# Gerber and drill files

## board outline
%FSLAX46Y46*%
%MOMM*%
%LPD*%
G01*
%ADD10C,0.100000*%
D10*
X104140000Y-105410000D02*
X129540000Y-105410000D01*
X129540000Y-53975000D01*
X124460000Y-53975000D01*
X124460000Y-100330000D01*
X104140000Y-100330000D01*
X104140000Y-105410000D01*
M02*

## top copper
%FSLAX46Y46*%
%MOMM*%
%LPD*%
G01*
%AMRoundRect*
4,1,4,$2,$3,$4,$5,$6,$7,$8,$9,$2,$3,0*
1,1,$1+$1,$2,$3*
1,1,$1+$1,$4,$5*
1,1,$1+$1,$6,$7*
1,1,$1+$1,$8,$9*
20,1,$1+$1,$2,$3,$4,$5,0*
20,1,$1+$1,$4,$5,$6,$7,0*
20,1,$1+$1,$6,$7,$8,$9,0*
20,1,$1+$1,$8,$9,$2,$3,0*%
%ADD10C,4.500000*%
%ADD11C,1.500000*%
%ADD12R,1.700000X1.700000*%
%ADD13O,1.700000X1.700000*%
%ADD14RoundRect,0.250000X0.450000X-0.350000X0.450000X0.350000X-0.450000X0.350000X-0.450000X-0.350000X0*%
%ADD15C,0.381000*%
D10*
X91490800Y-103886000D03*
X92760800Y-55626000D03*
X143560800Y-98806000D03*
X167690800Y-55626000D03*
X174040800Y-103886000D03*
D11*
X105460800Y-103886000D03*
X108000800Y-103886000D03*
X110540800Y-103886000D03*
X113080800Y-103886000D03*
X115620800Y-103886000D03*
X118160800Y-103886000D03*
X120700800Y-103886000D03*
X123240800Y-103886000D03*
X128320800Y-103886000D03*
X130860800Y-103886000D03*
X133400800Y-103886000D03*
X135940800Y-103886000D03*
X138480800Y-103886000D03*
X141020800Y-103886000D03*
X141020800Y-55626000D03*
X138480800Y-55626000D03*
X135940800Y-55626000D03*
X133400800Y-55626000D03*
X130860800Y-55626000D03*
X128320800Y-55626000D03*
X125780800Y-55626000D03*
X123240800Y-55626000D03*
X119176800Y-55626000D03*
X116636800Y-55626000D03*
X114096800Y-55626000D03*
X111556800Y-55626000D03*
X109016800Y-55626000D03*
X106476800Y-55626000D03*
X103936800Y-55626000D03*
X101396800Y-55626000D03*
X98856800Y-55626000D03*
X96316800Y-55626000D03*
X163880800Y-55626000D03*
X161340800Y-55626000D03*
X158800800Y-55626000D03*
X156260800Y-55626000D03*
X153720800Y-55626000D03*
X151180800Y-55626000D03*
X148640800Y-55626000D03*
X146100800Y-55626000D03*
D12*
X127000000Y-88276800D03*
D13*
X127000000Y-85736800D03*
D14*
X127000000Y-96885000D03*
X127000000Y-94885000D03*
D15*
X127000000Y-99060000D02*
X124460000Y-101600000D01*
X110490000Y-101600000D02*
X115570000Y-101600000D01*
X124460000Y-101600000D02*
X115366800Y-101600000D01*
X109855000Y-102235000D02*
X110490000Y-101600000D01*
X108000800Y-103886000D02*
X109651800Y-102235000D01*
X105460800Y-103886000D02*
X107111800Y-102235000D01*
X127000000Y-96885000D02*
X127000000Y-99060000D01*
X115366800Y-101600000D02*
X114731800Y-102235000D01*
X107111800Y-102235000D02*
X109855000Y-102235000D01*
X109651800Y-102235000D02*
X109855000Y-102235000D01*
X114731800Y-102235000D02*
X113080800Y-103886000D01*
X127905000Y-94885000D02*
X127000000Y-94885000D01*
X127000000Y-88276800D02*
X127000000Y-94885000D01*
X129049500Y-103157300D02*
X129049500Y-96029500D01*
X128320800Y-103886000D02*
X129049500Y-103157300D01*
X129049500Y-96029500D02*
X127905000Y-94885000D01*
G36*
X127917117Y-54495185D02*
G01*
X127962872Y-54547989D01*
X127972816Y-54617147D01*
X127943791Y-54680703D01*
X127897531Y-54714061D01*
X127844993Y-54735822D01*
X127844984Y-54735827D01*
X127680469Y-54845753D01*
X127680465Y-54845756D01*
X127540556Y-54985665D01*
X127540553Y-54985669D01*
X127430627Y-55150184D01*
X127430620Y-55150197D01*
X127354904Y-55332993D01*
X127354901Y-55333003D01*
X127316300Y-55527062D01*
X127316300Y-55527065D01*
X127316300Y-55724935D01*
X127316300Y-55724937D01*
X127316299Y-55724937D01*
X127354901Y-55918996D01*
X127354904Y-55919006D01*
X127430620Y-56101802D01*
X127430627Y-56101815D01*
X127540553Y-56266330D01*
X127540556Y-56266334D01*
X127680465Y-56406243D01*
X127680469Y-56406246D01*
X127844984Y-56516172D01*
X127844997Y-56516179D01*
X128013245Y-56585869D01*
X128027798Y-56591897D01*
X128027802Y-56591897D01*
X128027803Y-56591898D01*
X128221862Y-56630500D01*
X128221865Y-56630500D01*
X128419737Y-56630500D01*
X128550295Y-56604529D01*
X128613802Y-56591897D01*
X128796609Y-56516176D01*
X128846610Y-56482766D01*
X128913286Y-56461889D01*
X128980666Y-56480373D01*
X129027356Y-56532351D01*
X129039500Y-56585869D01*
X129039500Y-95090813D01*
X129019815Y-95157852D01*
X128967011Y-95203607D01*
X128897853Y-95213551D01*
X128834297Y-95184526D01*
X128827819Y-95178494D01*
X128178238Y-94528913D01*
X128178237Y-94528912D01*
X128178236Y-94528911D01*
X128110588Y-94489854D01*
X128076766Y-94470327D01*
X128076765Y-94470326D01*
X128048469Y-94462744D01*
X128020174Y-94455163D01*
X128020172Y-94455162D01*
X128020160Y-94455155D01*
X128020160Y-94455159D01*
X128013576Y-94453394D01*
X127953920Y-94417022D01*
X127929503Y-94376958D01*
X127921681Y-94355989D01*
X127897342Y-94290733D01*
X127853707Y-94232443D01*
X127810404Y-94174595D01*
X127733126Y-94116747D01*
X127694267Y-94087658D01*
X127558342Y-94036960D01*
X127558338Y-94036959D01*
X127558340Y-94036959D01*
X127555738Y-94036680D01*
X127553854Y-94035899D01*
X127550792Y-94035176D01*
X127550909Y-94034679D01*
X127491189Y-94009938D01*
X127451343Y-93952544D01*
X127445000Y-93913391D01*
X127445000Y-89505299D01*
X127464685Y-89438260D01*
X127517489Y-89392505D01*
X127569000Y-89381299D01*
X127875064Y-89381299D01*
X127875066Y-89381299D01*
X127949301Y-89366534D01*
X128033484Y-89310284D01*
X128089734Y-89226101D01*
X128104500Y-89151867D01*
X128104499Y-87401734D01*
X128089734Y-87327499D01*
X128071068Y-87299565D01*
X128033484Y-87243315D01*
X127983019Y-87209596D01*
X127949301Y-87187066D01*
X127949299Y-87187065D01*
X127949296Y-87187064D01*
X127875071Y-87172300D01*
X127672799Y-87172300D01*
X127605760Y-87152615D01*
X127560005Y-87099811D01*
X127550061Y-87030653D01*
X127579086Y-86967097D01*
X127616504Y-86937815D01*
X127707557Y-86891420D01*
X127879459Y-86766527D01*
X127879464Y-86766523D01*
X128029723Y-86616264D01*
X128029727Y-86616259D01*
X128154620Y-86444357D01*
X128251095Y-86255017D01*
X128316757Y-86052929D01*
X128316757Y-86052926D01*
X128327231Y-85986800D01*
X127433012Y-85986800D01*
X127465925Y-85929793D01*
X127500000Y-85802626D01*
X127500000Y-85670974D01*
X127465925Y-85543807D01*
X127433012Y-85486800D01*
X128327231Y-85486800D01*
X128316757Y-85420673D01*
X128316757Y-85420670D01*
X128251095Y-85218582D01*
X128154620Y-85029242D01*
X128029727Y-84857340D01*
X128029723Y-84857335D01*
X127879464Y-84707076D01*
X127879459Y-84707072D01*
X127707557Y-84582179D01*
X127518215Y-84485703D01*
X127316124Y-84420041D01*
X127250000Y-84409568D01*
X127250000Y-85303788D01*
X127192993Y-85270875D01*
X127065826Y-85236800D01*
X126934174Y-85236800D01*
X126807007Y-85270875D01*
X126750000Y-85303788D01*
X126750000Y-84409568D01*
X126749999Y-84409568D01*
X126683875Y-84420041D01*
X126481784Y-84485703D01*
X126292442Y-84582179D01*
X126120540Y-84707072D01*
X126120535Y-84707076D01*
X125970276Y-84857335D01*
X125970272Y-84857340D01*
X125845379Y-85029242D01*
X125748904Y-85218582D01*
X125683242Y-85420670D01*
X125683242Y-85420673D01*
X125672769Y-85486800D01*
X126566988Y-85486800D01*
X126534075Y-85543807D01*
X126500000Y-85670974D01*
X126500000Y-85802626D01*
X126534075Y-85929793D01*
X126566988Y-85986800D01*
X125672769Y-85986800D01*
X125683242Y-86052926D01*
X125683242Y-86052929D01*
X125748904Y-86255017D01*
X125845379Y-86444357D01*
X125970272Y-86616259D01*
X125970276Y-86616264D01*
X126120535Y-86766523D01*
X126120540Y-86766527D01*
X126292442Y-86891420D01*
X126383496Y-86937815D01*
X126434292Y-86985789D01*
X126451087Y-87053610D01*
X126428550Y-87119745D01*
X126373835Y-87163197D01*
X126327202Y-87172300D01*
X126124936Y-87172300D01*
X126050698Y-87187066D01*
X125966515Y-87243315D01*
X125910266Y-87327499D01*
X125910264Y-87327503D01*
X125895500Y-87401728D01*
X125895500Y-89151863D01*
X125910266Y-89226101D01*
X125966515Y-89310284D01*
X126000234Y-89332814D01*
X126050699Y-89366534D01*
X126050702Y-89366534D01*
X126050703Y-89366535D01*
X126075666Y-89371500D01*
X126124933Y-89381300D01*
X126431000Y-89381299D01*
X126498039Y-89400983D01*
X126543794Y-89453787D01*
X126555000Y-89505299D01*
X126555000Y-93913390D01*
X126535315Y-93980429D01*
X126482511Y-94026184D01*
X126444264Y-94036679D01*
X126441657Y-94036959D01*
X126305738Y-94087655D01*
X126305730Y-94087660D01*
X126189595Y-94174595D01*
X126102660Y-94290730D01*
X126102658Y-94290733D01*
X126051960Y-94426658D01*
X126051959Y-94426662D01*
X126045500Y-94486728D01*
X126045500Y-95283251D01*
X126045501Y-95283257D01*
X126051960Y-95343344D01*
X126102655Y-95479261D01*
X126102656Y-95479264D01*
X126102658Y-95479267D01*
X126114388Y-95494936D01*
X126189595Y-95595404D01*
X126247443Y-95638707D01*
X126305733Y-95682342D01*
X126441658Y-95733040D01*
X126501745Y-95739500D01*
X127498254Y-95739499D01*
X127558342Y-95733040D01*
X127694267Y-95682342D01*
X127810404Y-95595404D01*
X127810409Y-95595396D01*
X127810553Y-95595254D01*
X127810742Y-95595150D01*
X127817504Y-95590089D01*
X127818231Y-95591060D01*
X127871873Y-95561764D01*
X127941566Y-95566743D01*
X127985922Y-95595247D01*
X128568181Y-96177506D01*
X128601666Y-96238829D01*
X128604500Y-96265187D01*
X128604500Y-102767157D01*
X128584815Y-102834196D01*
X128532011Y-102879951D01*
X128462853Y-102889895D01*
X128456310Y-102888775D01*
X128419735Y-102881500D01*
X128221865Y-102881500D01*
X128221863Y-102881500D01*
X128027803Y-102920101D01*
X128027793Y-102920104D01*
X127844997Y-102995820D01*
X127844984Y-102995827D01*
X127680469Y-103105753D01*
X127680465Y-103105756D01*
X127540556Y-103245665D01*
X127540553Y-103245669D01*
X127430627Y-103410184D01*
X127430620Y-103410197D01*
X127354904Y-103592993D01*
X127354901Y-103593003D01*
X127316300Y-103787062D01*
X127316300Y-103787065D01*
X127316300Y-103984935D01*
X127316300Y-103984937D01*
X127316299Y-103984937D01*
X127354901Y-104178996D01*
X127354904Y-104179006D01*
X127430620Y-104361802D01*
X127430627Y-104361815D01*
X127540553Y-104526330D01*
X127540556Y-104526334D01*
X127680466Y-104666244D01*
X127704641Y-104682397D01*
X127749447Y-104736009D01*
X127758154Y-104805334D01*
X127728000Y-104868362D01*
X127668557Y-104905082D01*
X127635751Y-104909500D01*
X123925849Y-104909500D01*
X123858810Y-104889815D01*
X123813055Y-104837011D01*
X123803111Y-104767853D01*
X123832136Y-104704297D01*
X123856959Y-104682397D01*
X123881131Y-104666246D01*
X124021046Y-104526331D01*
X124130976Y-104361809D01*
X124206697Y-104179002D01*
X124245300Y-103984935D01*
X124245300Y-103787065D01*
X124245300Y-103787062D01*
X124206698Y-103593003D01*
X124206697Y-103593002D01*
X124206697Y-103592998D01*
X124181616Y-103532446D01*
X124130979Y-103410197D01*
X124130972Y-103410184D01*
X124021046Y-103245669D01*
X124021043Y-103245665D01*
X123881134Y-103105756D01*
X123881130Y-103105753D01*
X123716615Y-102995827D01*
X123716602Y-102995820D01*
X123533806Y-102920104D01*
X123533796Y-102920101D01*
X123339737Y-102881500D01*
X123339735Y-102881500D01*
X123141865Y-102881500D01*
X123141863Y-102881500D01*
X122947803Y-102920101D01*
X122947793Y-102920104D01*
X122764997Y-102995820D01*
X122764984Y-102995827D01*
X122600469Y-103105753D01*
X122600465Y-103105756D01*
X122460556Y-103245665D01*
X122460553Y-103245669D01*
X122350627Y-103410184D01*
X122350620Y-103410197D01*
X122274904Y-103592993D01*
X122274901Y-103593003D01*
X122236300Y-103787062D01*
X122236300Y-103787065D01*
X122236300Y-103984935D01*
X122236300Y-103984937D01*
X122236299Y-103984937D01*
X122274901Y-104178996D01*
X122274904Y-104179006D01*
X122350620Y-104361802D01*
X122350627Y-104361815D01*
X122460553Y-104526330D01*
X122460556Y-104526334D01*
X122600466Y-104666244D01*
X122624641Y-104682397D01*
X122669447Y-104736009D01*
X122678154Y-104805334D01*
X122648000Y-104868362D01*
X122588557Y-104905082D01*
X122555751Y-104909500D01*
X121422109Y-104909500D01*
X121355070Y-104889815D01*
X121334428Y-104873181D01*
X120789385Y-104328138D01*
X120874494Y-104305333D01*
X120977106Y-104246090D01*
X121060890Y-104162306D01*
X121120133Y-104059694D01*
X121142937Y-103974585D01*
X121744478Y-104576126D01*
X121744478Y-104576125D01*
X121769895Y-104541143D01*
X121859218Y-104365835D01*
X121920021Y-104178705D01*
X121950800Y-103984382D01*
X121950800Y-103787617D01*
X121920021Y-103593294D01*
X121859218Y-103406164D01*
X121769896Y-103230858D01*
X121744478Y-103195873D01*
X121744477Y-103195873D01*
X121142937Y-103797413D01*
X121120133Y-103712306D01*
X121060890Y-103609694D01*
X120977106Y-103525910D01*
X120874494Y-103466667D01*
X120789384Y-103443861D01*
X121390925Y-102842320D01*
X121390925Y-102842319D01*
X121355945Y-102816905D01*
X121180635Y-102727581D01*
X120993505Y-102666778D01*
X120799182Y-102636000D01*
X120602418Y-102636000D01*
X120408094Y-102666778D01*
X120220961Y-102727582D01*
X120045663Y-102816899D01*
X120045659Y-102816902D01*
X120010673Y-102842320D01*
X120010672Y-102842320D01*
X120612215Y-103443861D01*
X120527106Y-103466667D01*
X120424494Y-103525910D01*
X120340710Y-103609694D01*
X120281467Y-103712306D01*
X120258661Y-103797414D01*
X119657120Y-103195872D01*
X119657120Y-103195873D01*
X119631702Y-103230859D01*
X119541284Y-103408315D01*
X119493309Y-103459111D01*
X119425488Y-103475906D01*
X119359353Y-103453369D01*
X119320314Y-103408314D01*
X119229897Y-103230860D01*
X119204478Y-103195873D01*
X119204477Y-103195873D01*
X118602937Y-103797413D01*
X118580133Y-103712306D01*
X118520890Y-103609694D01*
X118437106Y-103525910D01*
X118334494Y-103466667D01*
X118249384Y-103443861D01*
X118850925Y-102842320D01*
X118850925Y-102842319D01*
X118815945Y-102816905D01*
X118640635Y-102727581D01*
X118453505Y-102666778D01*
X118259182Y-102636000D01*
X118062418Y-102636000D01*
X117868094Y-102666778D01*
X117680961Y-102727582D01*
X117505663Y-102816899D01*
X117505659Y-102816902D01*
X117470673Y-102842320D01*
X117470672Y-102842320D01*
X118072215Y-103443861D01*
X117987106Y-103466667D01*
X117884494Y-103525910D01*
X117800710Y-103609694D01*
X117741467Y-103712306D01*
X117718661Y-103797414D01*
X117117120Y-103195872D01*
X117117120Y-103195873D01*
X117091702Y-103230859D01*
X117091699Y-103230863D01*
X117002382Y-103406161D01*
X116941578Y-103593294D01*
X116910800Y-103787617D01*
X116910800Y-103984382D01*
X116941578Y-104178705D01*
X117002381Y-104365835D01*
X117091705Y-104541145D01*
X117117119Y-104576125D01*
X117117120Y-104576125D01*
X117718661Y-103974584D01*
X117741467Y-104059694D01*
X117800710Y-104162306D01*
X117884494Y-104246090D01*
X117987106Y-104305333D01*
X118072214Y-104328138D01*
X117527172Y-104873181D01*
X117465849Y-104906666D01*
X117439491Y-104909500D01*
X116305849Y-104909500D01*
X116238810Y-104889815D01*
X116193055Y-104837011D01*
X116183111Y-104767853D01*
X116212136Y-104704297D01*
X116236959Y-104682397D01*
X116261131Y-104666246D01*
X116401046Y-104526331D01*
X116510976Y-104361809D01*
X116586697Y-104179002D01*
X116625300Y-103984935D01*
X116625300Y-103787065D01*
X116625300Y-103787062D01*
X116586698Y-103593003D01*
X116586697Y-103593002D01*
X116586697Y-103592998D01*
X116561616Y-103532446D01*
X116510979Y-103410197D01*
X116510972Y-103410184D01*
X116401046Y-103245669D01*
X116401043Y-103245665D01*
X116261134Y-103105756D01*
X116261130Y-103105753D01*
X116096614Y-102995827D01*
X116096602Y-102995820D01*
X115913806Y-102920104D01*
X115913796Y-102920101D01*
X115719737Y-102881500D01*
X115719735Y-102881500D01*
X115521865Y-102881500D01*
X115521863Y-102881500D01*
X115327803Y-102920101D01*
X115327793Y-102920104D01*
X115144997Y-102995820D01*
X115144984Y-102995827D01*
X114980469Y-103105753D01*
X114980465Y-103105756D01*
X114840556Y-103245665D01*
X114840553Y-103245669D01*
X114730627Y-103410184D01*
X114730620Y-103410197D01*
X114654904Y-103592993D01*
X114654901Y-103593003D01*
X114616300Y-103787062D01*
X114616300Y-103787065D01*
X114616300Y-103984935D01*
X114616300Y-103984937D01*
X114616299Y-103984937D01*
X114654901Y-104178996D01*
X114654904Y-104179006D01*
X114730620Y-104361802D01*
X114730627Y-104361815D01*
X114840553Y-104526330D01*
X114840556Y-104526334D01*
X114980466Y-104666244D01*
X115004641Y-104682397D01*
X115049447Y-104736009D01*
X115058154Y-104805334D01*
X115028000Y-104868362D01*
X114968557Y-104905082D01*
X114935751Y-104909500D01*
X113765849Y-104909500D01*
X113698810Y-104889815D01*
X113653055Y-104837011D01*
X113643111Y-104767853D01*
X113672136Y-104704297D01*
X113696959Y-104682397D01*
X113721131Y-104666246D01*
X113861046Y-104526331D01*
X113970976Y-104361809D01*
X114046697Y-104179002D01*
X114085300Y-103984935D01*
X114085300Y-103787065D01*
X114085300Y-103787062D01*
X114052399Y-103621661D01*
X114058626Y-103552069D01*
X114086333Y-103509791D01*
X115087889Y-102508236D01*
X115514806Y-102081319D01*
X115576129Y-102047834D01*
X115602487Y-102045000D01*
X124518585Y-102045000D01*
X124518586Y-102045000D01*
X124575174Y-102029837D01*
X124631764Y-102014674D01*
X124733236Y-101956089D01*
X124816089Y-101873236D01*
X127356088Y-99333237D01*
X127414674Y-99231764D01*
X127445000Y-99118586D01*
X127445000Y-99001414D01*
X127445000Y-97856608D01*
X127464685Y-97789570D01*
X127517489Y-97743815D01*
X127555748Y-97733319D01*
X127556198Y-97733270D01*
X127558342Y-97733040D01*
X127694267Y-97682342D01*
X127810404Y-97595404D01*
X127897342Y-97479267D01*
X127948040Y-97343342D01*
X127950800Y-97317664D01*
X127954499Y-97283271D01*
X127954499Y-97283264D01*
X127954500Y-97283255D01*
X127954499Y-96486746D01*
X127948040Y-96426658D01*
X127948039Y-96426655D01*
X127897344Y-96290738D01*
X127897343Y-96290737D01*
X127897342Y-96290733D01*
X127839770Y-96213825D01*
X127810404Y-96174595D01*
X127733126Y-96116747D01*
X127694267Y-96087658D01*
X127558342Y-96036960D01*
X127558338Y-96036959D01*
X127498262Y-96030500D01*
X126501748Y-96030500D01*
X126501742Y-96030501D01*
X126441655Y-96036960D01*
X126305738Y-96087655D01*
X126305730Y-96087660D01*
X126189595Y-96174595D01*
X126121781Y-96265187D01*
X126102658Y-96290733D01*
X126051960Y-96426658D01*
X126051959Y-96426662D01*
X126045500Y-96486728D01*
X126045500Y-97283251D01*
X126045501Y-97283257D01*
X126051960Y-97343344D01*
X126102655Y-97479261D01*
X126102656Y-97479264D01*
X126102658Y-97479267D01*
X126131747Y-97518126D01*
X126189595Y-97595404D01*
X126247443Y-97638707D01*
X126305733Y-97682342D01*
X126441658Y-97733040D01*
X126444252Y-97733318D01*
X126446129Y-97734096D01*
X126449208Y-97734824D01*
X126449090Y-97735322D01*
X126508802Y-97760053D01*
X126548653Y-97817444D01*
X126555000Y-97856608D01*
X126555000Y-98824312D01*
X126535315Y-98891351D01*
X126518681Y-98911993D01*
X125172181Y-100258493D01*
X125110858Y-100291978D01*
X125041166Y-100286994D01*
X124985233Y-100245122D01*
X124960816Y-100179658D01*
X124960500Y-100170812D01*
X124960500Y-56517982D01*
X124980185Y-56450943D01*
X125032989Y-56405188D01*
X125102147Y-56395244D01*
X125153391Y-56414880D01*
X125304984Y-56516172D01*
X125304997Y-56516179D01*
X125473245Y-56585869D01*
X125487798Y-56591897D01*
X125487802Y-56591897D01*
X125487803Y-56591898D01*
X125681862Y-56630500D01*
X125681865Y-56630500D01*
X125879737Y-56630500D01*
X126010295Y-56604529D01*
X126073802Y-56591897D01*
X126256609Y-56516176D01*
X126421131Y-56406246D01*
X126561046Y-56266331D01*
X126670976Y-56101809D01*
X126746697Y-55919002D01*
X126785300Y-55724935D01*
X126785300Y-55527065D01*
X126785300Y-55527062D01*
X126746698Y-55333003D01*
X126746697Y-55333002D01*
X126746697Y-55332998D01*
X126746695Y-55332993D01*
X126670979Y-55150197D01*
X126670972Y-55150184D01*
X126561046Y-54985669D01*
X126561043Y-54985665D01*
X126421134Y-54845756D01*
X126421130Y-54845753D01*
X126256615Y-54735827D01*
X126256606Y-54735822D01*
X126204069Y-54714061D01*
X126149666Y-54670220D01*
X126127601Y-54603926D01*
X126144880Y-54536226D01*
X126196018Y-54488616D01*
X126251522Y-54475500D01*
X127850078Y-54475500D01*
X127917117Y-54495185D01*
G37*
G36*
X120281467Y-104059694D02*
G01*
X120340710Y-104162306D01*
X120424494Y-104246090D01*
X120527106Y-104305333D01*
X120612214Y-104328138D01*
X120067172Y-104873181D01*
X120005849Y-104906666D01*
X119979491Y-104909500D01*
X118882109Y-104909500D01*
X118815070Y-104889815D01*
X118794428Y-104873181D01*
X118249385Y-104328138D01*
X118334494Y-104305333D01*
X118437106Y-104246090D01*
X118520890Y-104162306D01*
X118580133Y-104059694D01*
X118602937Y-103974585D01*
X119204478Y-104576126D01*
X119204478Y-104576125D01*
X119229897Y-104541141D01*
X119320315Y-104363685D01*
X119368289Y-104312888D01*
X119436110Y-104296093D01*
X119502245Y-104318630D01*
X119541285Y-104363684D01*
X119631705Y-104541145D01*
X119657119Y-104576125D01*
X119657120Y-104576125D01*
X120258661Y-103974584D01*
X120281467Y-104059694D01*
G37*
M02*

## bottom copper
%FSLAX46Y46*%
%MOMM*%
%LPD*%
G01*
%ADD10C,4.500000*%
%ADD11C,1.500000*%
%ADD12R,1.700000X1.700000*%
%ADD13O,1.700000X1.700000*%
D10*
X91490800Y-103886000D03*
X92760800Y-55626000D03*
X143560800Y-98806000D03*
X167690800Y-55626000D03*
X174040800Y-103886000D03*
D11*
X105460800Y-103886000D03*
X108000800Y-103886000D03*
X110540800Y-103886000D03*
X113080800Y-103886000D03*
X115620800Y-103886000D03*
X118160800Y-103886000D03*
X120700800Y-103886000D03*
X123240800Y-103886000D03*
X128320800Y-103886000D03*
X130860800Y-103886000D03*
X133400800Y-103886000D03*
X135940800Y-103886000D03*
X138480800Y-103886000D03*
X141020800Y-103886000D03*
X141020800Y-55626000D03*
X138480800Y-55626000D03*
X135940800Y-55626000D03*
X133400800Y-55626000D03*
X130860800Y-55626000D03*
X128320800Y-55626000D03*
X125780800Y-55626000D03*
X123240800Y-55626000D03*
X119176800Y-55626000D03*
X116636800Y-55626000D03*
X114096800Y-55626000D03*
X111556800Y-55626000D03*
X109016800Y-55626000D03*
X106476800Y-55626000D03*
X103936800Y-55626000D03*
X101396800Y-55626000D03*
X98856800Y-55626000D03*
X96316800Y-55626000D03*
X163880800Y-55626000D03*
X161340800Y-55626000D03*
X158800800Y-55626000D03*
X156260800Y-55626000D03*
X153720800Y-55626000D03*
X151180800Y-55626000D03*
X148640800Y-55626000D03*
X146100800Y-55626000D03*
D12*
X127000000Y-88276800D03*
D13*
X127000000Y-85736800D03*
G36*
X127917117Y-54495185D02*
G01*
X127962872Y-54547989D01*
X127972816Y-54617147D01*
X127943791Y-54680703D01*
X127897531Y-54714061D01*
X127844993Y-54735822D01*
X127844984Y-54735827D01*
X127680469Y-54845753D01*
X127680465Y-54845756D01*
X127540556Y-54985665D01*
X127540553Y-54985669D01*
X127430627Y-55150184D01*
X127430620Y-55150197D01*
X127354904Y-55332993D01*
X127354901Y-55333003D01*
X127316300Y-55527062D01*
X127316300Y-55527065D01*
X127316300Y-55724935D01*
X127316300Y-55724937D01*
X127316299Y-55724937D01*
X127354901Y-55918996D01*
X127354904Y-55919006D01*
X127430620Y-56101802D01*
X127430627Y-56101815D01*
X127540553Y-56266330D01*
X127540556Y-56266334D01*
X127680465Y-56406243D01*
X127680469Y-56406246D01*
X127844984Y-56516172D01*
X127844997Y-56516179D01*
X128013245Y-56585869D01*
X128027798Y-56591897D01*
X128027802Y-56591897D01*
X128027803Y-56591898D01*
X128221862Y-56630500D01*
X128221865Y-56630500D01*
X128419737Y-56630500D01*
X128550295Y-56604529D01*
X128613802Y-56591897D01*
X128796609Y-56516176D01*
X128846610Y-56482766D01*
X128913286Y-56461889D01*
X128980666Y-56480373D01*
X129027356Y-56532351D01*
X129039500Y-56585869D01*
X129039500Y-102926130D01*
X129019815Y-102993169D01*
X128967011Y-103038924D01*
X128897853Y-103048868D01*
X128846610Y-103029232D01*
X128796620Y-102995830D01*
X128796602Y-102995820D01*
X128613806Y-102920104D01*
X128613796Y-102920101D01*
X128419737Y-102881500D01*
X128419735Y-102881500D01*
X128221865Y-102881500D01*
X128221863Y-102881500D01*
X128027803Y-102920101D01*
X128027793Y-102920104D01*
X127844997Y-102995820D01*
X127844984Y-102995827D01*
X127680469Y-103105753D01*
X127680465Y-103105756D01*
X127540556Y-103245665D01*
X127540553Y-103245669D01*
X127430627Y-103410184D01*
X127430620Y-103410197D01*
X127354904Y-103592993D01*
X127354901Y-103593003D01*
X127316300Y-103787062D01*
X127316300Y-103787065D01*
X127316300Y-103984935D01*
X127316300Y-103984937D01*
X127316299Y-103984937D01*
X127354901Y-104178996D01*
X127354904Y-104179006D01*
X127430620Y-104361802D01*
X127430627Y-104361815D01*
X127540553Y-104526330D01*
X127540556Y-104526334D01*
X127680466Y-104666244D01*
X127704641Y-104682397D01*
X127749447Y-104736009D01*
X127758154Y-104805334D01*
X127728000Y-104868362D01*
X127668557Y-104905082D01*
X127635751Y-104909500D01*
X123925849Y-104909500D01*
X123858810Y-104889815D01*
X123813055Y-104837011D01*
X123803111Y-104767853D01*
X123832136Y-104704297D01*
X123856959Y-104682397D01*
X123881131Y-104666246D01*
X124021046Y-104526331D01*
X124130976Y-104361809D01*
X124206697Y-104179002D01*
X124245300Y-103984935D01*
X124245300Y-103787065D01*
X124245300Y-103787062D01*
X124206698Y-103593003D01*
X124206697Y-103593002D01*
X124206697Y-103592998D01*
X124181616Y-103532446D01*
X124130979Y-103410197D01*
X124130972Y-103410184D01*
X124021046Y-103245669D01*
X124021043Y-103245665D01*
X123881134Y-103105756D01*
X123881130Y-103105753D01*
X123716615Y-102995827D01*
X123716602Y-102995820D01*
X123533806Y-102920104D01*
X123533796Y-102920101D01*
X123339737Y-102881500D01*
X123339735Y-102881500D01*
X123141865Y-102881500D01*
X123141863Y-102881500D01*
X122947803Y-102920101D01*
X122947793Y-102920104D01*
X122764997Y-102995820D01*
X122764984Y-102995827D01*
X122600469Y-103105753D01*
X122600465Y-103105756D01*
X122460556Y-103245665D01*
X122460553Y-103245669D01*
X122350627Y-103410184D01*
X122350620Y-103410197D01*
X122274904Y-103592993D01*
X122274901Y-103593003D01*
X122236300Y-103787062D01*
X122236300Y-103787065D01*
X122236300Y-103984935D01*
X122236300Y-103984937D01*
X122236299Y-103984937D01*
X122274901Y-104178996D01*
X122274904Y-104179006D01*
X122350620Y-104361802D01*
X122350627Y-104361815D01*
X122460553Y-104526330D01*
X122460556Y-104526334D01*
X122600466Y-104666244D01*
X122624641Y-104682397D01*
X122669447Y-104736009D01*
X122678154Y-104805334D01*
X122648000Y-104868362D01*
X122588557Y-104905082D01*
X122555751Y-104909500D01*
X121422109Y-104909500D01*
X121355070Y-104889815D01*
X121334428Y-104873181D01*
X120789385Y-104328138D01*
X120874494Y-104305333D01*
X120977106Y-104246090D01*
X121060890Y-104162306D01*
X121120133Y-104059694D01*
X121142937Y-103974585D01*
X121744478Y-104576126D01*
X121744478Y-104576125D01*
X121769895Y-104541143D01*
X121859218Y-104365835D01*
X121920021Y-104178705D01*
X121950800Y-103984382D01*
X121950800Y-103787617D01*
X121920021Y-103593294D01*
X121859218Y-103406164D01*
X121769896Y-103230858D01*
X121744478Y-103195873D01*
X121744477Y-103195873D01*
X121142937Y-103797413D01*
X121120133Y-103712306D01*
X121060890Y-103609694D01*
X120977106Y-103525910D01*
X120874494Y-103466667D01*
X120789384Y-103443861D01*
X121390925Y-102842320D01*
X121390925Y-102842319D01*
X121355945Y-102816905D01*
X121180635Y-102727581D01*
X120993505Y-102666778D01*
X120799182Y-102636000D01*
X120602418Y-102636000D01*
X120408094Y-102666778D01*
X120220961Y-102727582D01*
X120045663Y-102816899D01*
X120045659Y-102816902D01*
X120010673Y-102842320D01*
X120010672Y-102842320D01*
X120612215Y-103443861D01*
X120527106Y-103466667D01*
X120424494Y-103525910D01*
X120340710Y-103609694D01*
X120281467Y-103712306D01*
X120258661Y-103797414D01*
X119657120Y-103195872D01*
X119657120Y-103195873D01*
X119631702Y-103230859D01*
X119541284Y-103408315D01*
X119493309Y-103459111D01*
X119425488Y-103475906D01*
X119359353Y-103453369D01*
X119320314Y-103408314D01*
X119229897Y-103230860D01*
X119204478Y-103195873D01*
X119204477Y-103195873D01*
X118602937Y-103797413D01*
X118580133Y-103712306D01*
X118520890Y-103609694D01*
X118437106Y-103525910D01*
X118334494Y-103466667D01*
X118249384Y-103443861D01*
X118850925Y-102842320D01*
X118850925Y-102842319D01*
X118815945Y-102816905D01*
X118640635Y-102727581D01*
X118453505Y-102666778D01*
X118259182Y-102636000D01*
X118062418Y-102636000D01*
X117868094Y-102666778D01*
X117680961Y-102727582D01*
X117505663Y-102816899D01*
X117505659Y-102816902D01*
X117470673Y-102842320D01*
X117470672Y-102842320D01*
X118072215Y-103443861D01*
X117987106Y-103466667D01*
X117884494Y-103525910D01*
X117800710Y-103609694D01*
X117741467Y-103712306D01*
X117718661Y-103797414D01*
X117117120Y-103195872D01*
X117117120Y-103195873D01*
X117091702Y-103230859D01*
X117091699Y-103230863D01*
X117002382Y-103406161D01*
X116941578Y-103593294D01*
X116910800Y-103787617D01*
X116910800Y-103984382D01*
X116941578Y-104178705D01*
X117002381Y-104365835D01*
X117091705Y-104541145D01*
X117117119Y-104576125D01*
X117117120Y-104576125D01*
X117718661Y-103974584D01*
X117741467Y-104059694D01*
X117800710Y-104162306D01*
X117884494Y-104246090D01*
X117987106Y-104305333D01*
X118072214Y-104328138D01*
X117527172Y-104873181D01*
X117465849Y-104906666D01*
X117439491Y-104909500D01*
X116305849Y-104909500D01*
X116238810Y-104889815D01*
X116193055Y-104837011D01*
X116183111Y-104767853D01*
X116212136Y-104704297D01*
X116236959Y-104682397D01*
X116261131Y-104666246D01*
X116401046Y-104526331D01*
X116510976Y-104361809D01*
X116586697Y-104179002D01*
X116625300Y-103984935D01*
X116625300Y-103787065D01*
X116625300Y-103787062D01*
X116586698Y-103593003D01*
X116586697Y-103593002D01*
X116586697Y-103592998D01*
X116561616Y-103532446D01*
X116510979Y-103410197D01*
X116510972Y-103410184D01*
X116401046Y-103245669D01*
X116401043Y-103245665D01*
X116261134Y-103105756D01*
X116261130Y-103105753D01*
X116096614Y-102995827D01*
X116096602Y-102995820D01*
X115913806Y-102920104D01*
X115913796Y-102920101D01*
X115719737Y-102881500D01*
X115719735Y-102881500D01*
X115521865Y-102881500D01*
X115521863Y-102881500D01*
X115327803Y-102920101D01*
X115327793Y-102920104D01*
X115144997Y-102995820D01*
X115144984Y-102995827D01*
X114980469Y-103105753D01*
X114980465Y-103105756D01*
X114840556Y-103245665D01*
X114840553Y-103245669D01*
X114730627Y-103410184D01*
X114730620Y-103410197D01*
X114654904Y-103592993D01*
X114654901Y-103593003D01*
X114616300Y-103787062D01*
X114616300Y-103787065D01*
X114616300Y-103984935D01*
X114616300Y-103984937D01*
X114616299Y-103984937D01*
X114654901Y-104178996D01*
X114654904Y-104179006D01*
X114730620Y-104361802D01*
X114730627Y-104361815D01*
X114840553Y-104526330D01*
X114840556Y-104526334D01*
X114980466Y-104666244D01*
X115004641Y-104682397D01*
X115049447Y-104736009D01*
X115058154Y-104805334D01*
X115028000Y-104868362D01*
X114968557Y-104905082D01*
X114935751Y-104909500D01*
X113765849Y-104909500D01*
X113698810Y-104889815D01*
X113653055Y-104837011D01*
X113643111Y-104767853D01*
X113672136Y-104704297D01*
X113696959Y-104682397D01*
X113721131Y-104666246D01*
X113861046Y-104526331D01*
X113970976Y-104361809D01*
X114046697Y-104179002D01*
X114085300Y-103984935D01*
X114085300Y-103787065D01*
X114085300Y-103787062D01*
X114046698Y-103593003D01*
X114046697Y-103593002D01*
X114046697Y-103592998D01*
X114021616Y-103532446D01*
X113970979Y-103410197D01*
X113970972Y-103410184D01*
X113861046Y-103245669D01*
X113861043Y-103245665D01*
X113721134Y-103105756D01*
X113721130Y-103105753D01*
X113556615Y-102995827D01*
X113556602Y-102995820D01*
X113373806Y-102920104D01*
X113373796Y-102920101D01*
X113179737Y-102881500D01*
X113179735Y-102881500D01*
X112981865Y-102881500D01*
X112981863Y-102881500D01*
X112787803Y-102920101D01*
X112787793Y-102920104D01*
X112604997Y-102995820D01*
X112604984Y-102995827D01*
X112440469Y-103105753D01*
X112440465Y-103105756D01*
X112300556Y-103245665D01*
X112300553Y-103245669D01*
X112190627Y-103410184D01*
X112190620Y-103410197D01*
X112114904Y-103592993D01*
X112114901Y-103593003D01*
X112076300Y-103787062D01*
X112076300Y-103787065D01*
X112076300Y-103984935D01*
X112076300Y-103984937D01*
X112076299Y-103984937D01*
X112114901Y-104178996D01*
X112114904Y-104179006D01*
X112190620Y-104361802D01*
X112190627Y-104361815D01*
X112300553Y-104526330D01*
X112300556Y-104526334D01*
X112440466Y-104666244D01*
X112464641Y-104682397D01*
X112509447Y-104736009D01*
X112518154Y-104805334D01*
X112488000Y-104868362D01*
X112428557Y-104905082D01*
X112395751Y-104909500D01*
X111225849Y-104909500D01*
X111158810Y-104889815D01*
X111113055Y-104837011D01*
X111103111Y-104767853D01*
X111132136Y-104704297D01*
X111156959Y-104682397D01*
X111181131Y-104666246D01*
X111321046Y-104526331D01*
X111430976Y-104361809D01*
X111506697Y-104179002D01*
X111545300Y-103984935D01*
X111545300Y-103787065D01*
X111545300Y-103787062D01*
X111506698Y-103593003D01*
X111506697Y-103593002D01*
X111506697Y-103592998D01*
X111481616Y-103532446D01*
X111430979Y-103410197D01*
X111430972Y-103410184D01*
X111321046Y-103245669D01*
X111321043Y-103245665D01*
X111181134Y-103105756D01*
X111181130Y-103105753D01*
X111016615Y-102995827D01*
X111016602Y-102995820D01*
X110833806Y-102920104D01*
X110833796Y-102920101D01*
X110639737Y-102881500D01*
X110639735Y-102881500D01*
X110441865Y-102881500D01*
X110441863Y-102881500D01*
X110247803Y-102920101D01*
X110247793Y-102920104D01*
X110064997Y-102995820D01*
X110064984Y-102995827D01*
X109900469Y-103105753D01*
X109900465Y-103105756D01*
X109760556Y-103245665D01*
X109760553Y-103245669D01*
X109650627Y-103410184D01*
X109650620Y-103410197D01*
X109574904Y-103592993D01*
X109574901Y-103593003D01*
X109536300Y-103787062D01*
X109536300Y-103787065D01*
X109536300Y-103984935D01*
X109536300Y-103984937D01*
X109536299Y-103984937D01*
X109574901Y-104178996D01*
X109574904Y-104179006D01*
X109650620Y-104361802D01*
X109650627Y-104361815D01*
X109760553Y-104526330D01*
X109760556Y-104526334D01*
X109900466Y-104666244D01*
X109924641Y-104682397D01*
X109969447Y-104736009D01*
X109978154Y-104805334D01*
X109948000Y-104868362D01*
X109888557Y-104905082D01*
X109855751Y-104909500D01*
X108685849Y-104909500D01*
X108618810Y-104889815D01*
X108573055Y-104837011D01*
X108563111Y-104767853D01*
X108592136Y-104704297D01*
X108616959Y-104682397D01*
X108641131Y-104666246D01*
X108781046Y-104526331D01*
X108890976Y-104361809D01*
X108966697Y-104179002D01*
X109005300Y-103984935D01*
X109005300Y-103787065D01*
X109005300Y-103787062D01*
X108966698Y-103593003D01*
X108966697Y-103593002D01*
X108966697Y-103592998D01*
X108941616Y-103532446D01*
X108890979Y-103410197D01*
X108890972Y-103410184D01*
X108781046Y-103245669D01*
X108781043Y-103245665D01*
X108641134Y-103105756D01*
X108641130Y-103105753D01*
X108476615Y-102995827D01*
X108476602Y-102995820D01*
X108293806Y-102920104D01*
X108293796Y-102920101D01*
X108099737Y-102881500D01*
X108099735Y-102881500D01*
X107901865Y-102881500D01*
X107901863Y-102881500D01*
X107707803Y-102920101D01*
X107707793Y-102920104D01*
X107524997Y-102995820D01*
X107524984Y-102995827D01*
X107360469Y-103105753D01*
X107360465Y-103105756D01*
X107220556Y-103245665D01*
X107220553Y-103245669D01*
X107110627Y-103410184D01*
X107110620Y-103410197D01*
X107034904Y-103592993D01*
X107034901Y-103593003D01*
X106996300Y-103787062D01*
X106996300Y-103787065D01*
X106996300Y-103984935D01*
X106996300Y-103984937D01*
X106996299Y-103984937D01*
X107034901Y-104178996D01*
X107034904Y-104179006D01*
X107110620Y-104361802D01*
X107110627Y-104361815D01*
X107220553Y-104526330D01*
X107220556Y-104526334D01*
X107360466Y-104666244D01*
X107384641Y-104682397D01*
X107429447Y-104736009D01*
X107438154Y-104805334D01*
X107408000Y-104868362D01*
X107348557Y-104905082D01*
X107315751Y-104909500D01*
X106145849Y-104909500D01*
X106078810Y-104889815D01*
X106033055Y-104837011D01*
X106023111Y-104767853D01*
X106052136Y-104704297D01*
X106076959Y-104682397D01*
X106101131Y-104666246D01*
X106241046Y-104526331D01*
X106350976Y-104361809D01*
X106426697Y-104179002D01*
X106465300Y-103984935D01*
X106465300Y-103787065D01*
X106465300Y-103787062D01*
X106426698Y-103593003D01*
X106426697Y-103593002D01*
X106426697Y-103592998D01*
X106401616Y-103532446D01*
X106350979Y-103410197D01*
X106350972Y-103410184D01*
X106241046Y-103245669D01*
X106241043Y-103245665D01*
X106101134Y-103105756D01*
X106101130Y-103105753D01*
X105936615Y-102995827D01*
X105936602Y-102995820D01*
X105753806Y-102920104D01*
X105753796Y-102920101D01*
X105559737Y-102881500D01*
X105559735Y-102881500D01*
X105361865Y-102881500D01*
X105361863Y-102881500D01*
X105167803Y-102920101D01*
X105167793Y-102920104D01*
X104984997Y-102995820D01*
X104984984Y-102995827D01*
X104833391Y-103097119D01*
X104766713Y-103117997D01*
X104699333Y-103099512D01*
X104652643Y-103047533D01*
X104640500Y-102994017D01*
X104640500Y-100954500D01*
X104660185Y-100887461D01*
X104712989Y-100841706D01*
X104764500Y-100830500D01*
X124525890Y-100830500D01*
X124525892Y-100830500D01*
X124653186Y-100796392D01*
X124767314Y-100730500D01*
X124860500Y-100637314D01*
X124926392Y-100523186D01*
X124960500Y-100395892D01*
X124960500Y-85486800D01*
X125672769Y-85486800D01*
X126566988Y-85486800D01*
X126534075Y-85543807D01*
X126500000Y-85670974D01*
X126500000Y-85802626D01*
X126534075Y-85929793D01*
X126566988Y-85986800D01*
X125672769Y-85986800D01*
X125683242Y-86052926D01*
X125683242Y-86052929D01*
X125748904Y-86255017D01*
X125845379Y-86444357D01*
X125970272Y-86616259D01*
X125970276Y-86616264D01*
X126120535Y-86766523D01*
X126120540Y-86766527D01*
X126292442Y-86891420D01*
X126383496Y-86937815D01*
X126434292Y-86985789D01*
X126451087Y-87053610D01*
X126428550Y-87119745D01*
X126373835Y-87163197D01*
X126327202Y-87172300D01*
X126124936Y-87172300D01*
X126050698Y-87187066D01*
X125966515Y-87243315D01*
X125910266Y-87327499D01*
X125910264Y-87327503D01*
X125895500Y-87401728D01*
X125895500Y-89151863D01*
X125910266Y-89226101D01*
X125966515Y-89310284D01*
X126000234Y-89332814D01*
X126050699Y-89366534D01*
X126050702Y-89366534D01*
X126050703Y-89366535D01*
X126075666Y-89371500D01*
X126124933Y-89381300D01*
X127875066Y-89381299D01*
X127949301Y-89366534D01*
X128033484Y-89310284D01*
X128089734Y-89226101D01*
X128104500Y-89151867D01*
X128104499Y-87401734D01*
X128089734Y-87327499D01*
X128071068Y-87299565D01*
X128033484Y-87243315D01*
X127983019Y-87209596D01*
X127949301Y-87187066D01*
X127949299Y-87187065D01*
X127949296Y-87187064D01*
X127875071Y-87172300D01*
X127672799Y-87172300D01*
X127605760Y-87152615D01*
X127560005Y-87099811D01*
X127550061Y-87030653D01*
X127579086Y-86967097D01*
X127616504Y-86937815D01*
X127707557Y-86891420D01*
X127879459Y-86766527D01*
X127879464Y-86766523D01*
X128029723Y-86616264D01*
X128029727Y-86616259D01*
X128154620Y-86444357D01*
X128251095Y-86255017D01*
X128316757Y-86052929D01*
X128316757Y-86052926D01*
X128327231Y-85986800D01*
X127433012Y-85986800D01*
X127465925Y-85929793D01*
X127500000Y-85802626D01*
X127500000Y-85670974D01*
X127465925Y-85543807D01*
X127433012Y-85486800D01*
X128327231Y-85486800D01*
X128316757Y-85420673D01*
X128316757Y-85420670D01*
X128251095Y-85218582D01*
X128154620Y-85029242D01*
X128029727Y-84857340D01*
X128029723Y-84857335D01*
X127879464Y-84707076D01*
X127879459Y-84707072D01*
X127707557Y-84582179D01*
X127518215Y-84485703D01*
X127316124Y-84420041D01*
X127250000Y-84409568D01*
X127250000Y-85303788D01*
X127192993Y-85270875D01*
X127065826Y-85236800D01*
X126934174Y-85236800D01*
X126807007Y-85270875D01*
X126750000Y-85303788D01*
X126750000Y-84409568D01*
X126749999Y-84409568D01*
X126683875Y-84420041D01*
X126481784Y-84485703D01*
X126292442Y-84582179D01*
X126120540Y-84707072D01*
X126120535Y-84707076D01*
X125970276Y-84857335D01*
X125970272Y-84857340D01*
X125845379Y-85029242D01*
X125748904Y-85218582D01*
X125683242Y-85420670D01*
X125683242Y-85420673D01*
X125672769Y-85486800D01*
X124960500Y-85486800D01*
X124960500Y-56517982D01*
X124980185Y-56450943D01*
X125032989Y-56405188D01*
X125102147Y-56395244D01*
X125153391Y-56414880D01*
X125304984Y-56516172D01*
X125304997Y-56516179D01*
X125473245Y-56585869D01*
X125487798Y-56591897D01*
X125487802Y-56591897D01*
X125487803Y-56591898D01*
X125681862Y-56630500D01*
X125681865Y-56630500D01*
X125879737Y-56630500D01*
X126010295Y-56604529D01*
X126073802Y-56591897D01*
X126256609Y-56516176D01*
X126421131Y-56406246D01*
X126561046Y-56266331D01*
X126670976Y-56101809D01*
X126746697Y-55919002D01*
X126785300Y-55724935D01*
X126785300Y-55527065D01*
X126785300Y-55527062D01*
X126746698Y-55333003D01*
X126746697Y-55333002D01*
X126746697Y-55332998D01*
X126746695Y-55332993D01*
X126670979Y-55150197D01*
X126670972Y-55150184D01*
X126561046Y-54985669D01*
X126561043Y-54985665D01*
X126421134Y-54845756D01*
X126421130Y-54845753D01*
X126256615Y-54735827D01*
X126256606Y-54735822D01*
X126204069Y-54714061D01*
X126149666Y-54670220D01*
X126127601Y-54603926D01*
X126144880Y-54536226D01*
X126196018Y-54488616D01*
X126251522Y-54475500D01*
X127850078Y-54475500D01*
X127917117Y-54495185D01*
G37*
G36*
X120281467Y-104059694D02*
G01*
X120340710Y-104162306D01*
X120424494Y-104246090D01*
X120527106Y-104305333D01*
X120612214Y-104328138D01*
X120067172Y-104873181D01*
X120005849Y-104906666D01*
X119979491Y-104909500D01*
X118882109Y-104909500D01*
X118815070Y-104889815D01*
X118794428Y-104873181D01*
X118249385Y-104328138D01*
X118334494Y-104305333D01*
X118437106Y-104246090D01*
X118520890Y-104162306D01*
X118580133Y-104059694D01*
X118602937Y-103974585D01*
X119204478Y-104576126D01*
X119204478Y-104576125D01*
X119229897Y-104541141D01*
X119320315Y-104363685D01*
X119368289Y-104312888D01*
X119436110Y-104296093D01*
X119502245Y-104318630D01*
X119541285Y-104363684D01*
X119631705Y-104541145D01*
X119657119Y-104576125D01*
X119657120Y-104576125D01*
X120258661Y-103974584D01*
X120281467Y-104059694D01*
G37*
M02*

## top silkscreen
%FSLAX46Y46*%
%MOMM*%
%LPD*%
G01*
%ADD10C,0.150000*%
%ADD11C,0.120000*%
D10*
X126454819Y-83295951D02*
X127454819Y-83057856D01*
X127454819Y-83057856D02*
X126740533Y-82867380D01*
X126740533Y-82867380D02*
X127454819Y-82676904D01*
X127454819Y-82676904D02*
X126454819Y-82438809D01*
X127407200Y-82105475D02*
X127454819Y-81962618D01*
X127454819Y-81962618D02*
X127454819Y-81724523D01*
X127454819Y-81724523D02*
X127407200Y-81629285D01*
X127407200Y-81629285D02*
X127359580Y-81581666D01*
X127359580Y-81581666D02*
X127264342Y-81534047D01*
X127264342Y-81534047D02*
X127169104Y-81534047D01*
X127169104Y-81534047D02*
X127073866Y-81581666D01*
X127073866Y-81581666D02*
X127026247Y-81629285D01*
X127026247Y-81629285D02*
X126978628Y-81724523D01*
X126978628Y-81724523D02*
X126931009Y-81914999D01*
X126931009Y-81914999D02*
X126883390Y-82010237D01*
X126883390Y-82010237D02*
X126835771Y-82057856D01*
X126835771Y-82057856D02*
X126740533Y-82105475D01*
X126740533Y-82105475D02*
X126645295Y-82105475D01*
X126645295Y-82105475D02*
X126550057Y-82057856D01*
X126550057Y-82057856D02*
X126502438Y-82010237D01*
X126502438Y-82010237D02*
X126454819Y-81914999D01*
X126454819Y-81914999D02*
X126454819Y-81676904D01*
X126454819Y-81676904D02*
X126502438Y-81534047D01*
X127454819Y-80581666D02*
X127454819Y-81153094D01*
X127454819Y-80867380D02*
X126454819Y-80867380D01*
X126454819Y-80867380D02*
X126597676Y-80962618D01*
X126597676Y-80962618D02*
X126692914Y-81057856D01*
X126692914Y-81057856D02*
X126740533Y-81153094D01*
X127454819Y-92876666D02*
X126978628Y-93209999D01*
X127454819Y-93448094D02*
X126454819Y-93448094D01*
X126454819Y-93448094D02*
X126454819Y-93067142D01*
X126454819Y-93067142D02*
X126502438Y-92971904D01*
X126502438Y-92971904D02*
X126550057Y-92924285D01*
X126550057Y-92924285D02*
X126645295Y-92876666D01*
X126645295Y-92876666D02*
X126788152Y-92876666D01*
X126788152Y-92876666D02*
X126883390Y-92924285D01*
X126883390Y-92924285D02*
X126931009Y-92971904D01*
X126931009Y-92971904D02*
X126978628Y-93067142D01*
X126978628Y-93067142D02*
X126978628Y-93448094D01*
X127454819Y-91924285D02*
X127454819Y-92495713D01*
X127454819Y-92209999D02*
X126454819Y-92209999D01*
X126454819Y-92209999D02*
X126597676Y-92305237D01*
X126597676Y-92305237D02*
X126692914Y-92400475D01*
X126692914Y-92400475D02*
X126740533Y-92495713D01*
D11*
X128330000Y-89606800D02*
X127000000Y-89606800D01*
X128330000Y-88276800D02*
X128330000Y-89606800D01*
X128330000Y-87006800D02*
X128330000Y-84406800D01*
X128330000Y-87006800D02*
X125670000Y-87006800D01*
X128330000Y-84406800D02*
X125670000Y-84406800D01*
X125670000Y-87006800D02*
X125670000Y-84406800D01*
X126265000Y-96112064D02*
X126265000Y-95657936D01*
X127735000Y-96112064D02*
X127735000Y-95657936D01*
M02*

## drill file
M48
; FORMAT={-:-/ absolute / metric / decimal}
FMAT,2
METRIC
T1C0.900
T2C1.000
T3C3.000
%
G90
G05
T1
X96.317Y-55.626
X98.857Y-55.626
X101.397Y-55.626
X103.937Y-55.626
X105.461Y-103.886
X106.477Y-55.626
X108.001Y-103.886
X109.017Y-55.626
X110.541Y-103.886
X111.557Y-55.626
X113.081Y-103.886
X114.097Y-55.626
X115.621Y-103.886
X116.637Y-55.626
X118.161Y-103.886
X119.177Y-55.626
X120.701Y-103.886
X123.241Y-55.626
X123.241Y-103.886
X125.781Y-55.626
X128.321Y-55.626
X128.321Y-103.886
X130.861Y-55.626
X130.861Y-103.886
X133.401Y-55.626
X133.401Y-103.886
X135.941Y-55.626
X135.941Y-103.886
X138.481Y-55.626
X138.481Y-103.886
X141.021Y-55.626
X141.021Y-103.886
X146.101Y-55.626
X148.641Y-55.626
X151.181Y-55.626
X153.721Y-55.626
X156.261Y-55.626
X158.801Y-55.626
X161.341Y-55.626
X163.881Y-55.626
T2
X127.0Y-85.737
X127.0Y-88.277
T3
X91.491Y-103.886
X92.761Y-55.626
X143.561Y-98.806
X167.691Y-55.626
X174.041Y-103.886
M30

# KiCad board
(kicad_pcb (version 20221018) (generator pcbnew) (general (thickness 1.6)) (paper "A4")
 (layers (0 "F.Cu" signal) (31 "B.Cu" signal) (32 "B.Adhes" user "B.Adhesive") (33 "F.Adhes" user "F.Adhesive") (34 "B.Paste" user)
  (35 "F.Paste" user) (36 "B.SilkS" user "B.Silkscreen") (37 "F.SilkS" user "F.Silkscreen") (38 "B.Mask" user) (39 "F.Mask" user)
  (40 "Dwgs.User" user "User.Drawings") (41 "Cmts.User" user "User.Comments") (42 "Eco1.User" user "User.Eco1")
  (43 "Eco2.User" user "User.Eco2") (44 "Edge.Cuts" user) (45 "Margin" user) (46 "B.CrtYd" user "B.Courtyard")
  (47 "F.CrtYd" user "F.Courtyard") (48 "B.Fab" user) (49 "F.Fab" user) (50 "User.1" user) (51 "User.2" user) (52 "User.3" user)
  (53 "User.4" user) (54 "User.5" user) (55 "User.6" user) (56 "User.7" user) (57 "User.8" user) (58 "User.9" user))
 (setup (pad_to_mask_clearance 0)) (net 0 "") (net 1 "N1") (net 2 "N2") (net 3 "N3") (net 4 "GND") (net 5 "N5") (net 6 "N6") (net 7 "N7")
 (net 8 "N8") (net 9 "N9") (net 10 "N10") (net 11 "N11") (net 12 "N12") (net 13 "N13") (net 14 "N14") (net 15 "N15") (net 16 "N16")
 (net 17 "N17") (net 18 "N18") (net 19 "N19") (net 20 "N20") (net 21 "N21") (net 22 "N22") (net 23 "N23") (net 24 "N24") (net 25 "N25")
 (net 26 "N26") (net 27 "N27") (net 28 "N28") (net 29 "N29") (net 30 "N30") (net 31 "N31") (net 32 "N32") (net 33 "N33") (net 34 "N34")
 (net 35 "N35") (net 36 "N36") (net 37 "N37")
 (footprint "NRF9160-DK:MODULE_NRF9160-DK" (layer "F.Cu") (at 77.5208 48.007)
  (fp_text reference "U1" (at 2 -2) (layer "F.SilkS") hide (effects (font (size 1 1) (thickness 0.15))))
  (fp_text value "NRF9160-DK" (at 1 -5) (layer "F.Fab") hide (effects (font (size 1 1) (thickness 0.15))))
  (pad "" thru_hole circle (at 13.97 55.879) (size 4.5 4.5) (drill 3) (layers "*.Cu" "*.Mask"))
  (pad "" thru_hole circle (at 15.24 7.619) (size 4.5 4.5) (drill 3) (layers "*.Cu" "*.Mask"))
  (pad "" thru_hole circle (at 66.04 50.799) (size 4.5 4.5) (drill 3) (layers "*.Cu" "*.Mask"))
  (pad "" thru_hole circle (at 90.17 7.619) (size 4.5 4.5) (drill 3) (layers "*.Cu" "*.Mask"))
  (pad "" thru_hole circle (at 96.52 55.879) (size 4.5 4.5) (drill 3) (layers "*.Cu" "*.Mask"))
  (pad "P1_1" thru_hole circle (at 27.94 55.879) (size 1.5 1.5) (drill 0.9) (layers "*.Cu" "*.Mask") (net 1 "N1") (solder_mask_margin 0.102))
  (pad "P1_2" thru_hole circle (at 30.48 55.879) (size 1.5 1.5) (drill 0.9) (layers "*.Cu" "*.Mask") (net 1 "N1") (solder_mask_margin 0.102))
  (pad "P1_3" thru_hole circle (at 33.02 55.879) (size 1.5 1.5) (drill 0.9) (layers "*.Cu" "*.Mask") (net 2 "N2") (solder_mask_margin 0.102))
  (pad "P1_4" thru_hole circle (at 35.56 55.879) (size 1.5 1.5) (drill 0.9) (layers "*.Cu" "*.Mask") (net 1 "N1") (solder_mask_margin 0.102))
  (pad "P1_5" thru_hole circle (at 38.1 55.879) (size 1.5 1.5) (drill 0.9) (layers "*.Cu" "*.Mask") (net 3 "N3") (solder_mask_margin 0.102))
  (pad "P1_6" thru_hole circle (at 40.64 55.879) (size 1.5 1.5) (drill 0.9) (layers "*.Cu" "*.Mask") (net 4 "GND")
   (solder_mask_margin 0.102))
  (pad "P1_7" thru_hole circle (at 43.18 55.879) (size 1.5 1.5) (drill 0.9) (layers "*.Cu" "*.Mask") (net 4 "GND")
   (solder_mask_margin 0.102))
  (pad "P1_8" thru_hole circle (at 45.72 55.879) (size 1.5 1.5) (drill 0.9) (layers "*.Cu" "*.Mask") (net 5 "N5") (solder_mask_margin 0.102))
  (pad "P2_1" thru_hole circle (at 50.8 55.879) (size 1.5 1.5) (drill 0.9) (layers "*.Cu" "*.Mask") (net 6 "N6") (solder_mask_margin 0.102))
  (pad "P2_2" thru_hole circle (at 53.34 55.879) (size 1.5 1.5) (drill 0.9) (layers "*.Cu" "*.Mask") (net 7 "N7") (solder_mask_margin 0.102))
  (pad "P2_3" thru_hole circle (at 55.88 55.879) (size 1.5 1.5) (drill 0.9) (layers "*.Cu" "*.Mask") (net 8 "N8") (solder_mask_margin 0.102))
  (pad "P2_4" thru_hole circle (at 58.42 55.879) (size 1.5 1.5) (drill 0.9) (layers "*.Cu" "*.Mask") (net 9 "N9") (solder_mask_margin 0.102))
  (pad "P2_5" thru_hole circle (at 60.96 55.879) (size 1.5 1.5) (drill 0.9) (layers "*.Cu" "*.Mask") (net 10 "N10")
   (solder_mask_margin 0.102))
  (pad "P2_6" thru_hole circle (at 63.5 55.879) (size 1.5 1.5) (drill 0.9) (layers "*.Cu" "*.Mask") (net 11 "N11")
   (solder_mask_margin 0.102))
  (pad "P3_1" thru_hole circle (at 63.5 7.619) (size 1.5 1.5) (drill 0.9) (layers "*.Cu" "*.Mask") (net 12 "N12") (solder_mask_margin 0.102))
  (pad "P3_2" thru_hole circle (at 60.96 7.619) (size 1.5 1.5) (drill 0.9) (layers "*.Cu" "*.Mask") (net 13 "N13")
   (solder_mask_margin 0.102))
  (pad "P3_3" thru_hole circle (at 58.42 7.619) (size 1.5 1.5) (drill 0.9) (layers "*.Cu" "*.Mask") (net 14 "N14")
   (solder_mask_margin 0.102))
  (pad "P3_4" thru_hole circle (at 55.88 7.619) (size 1.5 1.5) (drill 0.9) (layers "*.Cu" "*.Mask") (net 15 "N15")
   (solder_mask_margin 0.102))
  (pad "P3_5" thru_hole circle (at 53.34 7.619) (size 1.5 1.5) (drill 0.9) (layers "*.Cu" "*.Mask") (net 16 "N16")
   (solder_mask_margin 0.102))
  (pad "P3_6" thru_hole circle (at 50.8 7.619) (size 1.5 1.5) (drill 0.9) (layers "*.Cu" "*.Mask") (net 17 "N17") (solder_mask_margin 0.102))
  (pad "P3_7" thru_hole circle (at 48.26 7.619) (size 1.5 1.5) (drill 0.9) (layers "*.Cu" "*.Mask") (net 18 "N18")
   (solder_mask_margin 0.102))
  (pad "P3_8" thru_hole circle (at 45.72 7.619) (size 1.5 1.5) (drill 0.9) (layers "*.Cu" "*.Mask") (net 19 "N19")
   (solder_mask_margin 0.102))
  (pad "P4_1" thru_hole circle (at 41.656 7.619) (size 1.5 1.5) (drill 0.9) (layers "*.Cu" "*.Mask") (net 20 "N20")
   (solder_mask_margin 0.102))
  (pad "P4_2" thru_hole circle (at 39.116 7.619) (size 1.5 1.5) (drill 0.9) (layers "*.Cu" "*.Mask") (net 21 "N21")
   (solder_mask_margin 0.102))
  (pad "P4_3" thru_hole circle (at 36.576 7.619) (size 1.5 1.5) (drill 0.9) (layers "*.Cu" "*.Mask") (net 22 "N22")
   (solder_mask_margin 0.102))
  (pad "P4_4" thru_hole circle (at 34.036 7.619) (size 1.5 1.5) (drill 0.9) (layers "*.Cu" "*.Mask") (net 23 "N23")
   (solder_mask_margin 0.102))
  (pad "P4_5" thru_hole circle (at 31.496 7.619) (size 1.5 1.5) (drill 0.9) (layers "*.Cu" "*.Mask") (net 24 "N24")
   (solder_mask_margin 0.102))
  (pad "P4_6" thru_hole circle (at 28.956 7.619) (size 1.5 1.5) (drill 0.9) (layers "*.Cu" "*.Mask") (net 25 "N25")
   (solder_mask_margin 0.102))
  (pad "P4_7" thru_hole circle (at 26.416 7.619) (size 1.5 1.5) (drill 0.9) (layers "*.Cu" "*.Mask") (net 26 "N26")
   (solder_mask_margin 0.102))
  (pad "P4_8" thru_hole circle (at 23.876 7.619) (size 1.5 1.5) (drill 0.9) (layers "*.Cu" "*.Mask") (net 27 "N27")
   (solder_mask_margin 0.102))
  (pad "P4_9" thru_hole circle (at 21.336 7.619) (size 1.5 1.5) (drill 0.9) (layers "*.Cu" "*.Mask") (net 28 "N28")
   (solder_mask_margin 0.102))
  (pad "P4_10" thru_hole circle (at 18.796 7.619) (size 1.5 1.5) (drill 0.9) (layers "*.Cu" "*.Mask") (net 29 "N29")
   (solder_mask_margin 0.102))
  (pad "P6_1" thru_hole circle (at 86.36 7.619) (size 1.5 1.5) (drill 0.9) (layers "*.Cu" "*.Mask") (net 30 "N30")
   (solder_mask_margin 0.102))
  (pad "P6_2" thru_hole circle (at 83.82 7.619) (size 1.5 1.5) (drill 0.9) (layers "*.Cu" "*.Mask") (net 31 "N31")
   (solder_mask_margin 0.102))
  (pad "P6_3" thru_hole circle (at 81.28 7.619) (size 1.5 1.5) (drill 0.9) (layers "*.Cu" "*.Mask") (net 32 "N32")
   (solder_mask_margin 0.102))
  (pad "P6_4" thru_hole circle (at 78.74 7.619) (size 1.5 1.5) (drill 0.9) (layers "*.Cu" "*.Mask") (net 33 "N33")
   (solder_mask_margin 0.102))
  (pad "P6_5" thru_hole circle (at 76.2 7.619) (size 1.5 1.5) (drill 0.9) (layers "*.Cu" "*.Mask") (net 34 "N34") (solder_mask_margin 0.102))
  (pad "P6_6" thru_hole circle (at 73.66 7.619) (size 1.5 1.5) (drill 0.9) (layers "*.Cu" "*.Mask") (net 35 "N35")
   (solder_mask_margin 0.102))
  (pad "P6_7" thru_hole circle (at 71.12 7.619) (size 1.5 1.5) (drill 0.9) (layers "*.Cu" "*.Mask") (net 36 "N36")
   (solder_mask_margin 0.102))
  (pad "P6_8" thru_hole circle (at 68.58 7.619) (size 1.5 1.5) (drill 0.9) (layers "*.Cu" "*.Mask") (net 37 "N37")
   (solder_mask_margin 0.102)))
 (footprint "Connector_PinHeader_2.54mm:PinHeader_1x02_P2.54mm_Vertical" (layer "F.Cu") (at 127 88.2768 180)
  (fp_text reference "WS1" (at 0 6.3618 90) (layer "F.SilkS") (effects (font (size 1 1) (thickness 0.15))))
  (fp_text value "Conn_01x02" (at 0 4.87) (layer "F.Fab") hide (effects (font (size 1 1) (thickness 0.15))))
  (fp_line (start -1.33 -1.33) (end 0 -1.33) (stroke (width 0.12) (type solid)) (layer "F.SilkS"))
  (fp_line (start -1.33 0) (end -1.33 -1.33) (stroke (width 0.12) (type solid)) (layer "F.SilkS"))
  (fp_line (start -1.33 1.27) (end -1.33 3.87) (stroke (width 0.12) (type solid)) (layer "F.SilkS"))
  (fp_line (start -1.33 1.27) (end 1.33 1.27) (stroke (width 0.12) (type solid)) (layer "F.SilkS"))
  (fp_line (start -1.33 3.87) (end 1.33 3.87) (stroke (width 0.12) (type solid)) (layer "F.SilkS"))
  (fp_line (start 1.33 1.27) (end 1.33 3.87) (stroke (width 0.12) (type solid)) (layer "F.SilkS"))
  (pad "1" thru_hole rect (at 0 0 180) (size 1.7 1.7) (drill 1) (layers "*.Cu" "*.Mask") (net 6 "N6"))
  (pad "2" thru_hole oval (at 0 2.54 180) (size 1.7 1.7) (drill 1) (layers "*.Cu" "*.Mask") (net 4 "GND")))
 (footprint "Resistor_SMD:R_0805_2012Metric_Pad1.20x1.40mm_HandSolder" (layer "F.Cu") (at 127 95.885 90)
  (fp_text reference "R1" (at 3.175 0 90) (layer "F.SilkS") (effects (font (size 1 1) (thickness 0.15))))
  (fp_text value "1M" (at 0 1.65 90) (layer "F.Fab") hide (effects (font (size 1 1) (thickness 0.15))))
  (fp_line (start -0.227064 -0.735) (end 0.227064 -0.735) (stroke (width 0.12) (type solid)) (layer "F.SilkS"))
  (fp_line (start -0.227064 0.735) (end 0.227064 0.735) (stroke (width 0.12) (type solid)) (layer "F.SilkS"))
  (pad "1" smd roundrect (at -1 0 90) (size 1.2 1.4) (layers "F.Cu" "F.Paste" "F.Mask") (roundrect_rratio 0.2083333333) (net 1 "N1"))
  (pad "2" smd roundrect (at 1 0 90) (size 1.2 1.4) (layers "F.Cu" "F.Paste" "F.Mask") (roundrect_rratio 0.2083333333) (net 6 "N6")))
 (gr_poly
  (pts (xy 104.14 105.41) (xy 129.54 105.41) (xy 129.54 53.975) (xy 124.46 53.975) (xy 124.46 100.33) (xy 104.14 100.33))
  (stroke (width 0.1) (type solid)) (fill none) (layer "Edge.Cuts"))
 (segment (start 127 99.06) (end 124.46 101.6) (width 0.381) (layer "F.Cu") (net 1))
 (segment (start 110.49 101.6) (end 115.57 101.6) (width 0.381) (layer "F.Cu") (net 1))
 (segment (start 124.46 101.6) (end 115.3668 101.6) (width 0.381) (layer "F.Cu") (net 1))
 (segment (start 109.855 102.235) (end 110.49 101.6) (width 0.381) (layer "F.Cu") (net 1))
 (segment (start 108.0008 103.886) (end 109.6518 102.235) (width 0.381) (layer "F.Cu") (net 1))
 (segment (start 105.4608 103.886) (end 107.1118 102.235) (width 0.381) (layer "F.Cu") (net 1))
 (segment (start 127 96.885) (end 127 99.06) (width 0.381) (layer "F.Cu") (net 1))
 (segment (start 115.3668 101.6) (end 114.7318 102.235) (width 0.381) (layer "F.Cu") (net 1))
 (segment (start 107.1118 102.235) (end 109.855 102.235) (width 0.381) (layer "F.Cu") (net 1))
 (segment (start 109.6518 102.235) (end 109.855 102.235) (width 0.381) (layer "F.Cu") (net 1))
 (segment (start 114.7318 102.235) (end 113.0808 103.886) (width 0.381) (layer "F.Cu") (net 1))
 (segment (start 127.905 94.885) (end 127 94.885) (width 0.381) (layer "F.Cu") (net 6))
 (segment (start 127 88.2768) (end 127 94.885) (width 0.381) (layer "F.Cu") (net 6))
 (segment (start 129.0495 103.1573) (end 129.0495 96.0295) (width 0.381) (layer "F.Cu") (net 6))
 (segment (start 128.3208 103.886) (end 129.0495 103.1573) (width 0.381) (layer "F.Cu") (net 6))
 (segment (start 129.0495 96.0295) (end 127.905 94.885) (width 0.381) (layer "F.Cu") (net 6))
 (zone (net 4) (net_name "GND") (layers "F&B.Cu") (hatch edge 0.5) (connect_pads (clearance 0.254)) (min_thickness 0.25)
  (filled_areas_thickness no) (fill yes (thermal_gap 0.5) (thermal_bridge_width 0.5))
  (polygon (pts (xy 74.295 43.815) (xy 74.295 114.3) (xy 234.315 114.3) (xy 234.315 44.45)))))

